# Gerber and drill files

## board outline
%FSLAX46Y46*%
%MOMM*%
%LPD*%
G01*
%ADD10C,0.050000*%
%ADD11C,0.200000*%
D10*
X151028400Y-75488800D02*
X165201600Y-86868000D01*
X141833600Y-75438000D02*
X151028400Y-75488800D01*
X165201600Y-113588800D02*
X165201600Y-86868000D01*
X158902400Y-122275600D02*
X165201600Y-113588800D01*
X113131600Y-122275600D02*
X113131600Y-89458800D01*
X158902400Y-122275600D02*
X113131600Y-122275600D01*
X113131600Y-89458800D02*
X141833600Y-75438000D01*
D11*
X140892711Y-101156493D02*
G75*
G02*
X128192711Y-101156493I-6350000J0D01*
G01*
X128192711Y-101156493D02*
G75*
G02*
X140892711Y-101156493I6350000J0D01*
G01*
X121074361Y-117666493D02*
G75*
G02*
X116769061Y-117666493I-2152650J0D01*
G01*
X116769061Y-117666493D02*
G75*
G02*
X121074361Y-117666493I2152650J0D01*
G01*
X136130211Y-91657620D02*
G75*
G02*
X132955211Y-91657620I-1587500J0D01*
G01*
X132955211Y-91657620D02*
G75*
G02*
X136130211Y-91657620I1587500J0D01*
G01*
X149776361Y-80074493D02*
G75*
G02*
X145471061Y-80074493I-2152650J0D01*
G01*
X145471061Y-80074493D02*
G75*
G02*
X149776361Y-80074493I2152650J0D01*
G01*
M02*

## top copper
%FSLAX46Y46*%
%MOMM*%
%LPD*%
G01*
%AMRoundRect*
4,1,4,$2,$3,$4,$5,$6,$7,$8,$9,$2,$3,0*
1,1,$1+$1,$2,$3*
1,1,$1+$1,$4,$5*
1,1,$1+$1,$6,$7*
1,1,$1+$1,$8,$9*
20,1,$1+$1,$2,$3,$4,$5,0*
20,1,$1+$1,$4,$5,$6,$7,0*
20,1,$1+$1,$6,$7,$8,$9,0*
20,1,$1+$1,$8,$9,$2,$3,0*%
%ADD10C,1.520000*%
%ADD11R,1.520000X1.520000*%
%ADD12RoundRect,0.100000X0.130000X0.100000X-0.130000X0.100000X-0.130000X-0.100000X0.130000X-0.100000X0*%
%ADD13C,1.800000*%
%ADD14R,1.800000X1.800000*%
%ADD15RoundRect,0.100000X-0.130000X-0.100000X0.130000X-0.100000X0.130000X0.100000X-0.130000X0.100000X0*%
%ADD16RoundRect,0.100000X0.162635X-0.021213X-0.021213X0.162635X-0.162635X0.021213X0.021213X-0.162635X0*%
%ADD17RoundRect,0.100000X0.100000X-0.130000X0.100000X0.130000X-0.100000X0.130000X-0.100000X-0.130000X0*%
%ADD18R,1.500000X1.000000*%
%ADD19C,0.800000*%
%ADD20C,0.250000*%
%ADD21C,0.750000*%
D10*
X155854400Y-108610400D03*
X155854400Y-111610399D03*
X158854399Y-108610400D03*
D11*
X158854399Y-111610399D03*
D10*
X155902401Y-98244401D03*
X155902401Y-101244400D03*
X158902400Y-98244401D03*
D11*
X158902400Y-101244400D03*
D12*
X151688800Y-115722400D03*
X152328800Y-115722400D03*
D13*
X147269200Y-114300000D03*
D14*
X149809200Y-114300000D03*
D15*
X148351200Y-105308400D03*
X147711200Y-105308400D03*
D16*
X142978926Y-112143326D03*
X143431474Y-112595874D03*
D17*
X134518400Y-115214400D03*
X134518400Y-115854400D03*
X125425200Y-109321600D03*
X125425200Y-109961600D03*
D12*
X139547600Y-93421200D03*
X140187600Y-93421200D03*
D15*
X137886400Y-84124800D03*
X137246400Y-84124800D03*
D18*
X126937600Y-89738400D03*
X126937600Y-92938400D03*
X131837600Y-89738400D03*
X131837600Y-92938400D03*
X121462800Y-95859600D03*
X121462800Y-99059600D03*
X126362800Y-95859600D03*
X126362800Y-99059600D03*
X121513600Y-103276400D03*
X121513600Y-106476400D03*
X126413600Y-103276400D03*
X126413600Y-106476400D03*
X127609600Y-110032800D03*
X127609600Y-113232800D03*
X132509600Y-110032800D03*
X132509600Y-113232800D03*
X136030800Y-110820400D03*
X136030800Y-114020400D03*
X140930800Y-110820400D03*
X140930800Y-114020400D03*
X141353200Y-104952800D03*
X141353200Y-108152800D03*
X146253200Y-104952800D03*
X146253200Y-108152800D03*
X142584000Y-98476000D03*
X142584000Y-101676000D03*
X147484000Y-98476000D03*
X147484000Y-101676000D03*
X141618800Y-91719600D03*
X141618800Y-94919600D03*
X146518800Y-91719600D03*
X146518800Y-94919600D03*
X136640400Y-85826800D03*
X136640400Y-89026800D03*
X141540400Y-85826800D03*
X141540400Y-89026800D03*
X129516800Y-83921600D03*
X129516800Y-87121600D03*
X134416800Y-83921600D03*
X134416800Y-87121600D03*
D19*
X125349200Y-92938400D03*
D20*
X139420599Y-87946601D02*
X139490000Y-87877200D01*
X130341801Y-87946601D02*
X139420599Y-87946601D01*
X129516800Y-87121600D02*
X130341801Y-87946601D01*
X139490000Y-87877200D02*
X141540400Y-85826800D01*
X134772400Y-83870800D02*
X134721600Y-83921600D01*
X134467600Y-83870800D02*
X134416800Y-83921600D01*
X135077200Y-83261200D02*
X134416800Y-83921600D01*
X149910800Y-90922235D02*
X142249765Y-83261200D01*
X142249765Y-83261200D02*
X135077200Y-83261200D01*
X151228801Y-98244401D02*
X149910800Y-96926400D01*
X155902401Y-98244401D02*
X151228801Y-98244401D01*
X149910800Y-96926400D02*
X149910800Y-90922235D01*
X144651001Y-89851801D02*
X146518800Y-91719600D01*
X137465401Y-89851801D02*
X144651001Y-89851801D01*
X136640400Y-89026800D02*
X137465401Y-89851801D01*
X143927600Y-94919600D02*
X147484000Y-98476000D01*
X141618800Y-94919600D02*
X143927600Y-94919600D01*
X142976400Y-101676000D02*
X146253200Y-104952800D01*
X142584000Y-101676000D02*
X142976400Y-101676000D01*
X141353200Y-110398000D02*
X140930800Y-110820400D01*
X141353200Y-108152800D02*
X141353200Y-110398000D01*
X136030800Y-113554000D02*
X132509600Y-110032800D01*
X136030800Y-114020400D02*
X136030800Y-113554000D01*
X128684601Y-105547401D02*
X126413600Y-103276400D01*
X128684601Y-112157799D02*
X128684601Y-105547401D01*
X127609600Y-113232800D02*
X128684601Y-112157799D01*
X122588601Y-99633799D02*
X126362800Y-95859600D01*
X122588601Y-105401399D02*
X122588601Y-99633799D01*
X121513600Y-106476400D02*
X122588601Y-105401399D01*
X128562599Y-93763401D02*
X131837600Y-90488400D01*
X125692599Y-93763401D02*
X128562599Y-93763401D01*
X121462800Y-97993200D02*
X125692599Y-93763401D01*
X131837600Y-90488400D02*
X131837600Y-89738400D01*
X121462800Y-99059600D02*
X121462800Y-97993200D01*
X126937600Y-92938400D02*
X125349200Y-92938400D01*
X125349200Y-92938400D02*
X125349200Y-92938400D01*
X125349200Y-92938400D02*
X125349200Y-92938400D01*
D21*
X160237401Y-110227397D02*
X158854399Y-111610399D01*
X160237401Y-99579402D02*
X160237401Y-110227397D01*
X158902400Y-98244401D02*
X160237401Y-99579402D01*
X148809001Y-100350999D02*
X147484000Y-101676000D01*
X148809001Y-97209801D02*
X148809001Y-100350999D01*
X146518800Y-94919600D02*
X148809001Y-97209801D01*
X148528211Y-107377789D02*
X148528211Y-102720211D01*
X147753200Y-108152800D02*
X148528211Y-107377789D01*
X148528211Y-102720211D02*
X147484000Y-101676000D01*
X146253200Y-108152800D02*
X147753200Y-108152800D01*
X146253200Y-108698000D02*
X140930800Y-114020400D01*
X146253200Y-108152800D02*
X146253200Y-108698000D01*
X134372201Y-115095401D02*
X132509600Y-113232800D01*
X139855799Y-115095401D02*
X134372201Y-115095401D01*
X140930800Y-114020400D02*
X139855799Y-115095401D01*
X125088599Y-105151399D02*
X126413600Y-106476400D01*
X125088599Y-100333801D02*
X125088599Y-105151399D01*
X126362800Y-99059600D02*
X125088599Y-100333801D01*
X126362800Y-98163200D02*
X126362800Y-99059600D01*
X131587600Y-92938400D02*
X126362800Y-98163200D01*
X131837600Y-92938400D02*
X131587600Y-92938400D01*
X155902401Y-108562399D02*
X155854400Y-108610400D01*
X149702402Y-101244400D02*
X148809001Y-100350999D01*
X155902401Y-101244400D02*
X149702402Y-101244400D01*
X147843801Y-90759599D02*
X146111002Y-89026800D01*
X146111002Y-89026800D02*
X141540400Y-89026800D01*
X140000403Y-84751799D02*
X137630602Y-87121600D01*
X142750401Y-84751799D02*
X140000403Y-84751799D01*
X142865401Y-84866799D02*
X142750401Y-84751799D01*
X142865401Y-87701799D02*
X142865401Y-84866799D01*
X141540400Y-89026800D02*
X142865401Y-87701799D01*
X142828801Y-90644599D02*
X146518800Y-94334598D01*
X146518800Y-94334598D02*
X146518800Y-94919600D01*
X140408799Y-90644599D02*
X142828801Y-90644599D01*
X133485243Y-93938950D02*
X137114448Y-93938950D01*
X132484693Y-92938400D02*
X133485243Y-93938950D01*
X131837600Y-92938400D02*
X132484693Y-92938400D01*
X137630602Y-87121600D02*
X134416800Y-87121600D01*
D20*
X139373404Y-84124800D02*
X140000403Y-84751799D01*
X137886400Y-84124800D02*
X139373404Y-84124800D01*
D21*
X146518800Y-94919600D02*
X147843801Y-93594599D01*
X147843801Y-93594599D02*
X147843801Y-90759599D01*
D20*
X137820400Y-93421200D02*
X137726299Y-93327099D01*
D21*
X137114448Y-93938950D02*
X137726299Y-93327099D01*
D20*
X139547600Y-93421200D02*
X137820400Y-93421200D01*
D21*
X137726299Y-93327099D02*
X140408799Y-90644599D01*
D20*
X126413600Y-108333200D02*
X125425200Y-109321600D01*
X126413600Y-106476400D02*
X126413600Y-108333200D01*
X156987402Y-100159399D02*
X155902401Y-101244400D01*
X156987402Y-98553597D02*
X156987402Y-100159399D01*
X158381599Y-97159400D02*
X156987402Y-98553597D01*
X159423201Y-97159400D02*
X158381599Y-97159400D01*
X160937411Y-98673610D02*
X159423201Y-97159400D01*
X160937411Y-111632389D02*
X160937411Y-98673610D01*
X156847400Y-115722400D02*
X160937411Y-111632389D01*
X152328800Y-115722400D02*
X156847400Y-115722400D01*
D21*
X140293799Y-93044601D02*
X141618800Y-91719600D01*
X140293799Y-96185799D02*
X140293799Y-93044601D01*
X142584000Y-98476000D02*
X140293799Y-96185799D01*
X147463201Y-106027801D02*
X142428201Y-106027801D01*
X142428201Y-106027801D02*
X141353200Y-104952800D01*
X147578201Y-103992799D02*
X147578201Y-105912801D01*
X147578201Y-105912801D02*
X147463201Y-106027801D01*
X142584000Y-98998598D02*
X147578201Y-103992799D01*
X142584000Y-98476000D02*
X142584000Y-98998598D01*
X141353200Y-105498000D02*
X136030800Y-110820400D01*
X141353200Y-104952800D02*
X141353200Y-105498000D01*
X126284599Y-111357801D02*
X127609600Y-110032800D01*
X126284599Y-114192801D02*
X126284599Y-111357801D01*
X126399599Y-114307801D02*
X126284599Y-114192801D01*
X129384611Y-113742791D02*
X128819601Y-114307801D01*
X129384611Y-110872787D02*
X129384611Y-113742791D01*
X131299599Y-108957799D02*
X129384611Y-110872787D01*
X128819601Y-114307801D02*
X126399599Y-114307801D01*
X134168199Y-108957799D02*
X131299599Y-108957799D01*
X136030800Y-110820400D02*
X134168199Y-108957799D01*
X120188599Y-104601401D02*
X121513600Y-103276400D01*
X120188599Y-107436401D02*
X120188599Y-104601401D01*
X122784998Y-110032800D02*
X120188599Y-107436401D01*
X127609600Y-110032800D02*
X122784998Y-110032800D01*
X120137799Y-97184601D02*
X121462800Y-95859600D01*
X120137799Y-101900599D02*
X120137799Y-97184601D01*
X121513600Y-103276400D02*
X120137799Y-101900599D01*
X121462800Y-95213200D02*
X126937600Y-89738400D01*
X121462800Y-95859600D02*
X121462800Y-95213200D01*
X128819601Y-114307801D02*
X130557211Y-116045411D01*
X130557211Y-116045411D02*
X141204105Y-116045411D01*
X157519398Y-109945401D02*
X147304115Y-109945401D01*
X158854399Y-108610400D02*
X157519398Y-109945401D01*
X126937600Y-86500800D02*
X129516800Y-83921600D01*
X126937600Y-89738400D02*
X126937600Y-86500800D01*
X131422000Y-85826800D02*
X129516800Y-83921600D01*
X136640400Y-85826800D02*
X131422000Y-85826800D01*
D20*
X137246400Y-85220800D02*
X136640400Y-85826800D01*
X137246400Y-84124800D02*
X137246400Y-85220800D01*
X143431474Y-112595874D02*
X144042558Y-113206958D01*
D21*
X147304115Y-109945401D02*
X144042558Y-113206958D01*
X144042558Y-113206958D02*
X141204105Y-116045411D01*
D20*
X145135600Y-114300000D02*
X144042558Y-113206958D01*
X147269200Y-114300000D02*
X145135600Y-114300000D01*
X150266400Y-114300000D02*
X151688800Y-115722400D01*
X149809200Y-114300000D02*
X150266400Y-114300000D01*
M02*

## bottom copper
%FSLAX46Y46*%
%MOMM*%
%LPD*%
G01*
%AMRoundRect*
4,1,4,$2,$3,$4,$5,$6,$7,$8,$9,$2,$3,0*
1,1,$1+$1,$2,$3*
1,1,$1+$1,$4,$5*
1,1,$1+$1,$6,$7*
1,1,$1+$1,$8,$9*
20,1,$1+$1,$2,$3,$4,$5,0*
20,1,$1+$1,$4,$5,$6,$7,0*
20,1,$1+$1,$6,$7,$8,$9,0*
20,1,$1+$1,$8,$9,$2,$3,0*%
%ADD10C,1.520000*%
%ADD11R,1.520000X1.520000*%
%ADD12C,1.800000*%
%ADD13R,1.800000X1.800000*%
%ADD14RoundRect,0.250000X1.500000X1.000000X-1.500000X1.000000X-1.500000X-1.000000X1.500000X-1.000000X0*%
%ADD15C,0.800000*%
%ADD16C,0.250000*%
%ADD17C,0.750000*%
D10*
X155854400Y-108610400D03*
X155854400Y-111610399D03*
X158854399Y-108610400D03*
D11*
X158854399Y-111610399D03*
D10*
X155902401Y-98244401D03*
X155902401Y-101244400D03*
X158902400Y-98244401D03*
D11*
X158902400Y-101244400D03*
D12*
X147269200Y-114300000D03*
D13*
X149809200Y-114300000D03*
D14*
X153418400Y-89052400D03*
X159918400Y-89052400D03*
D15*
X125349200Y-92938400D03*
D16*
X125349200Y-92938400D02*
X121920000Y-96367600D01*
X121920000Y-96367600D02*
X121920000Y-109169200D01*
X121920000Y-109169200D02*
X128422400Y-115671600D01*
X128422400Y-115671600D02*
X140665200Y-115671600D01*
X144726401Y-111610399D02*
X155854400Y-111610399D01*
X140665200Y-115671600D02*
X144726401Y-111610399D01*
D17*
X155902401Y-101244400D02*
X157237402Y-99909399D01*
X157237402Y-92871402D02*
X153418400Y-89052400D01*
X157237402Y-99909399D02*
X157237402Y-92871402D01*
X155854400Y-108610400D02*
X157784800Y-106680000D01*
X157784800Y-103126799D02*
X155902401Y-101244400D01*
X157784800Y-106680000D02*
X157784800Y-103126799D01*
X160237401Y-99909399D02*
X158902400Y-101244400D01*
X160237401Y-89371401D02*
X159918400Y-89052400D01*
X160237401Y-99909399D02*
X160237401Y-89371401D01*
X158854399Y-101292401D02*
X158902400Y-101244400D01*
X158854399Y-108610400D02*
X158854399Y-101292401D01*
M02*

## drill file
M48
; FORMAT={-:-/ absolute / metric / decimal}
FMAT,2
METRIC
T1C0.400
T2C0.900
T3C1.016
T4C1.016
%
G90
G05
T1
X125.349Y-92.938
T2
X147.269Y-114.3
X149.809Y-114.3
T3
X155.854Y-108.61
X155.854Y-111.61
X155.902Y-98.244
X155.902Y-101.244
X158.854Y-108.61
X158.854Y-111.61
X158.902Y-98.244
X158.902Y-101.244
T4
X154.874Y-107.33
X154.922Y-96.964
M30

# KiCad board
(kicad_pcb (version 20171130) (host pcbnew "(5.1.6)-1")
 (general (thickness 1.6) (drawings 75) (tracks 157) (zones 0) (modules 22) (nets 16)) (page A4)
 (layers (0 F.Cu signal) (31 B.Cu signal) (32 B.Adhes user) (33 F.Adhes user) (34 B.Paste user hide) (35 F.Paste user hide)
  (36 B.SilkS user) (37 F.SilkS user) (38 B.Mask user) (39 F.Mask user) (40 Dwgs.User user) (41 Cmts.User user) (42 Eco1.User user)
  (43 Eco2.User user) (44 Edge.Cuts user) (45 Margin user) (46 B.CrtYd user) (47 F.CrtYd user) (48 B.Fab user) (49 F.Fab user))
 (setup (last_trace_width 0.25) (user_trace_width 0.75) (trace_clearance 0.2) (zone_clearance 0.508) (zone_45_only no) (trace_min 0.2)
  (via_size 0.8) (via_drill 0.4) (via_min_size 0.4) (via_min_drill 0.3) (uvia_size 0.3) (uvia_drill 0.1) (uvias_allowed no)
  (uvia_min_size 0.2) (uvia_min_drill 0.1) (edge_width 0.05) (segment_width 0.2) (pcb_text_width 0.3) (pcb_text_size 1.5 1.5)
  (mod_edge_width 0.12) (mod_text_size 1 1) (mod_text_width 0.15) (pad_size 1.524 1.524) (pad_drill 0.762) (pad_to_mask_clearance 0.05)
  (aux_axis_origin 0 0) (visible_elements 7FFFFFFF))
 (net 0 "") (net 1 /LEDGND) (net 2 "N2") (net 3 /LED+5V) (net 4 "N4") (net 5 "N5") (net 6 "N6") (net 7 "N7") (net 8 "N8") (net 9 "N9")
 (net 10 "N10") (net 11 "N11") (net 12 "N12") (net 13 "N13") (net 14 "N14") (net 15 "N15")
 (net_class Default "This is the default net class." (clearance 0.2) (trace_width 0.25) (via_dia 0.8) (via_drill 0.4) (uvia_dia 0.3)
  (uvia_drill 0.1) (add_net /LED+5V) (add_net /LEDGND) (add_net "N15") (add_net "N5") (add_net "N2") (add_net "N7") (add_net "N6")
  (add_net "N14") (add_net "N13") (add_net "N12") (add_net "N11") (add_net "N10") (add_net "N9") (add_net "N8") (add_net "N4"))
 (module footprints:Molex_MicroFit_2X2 (layer B.Cu) (at 158.854399 111.610399 270)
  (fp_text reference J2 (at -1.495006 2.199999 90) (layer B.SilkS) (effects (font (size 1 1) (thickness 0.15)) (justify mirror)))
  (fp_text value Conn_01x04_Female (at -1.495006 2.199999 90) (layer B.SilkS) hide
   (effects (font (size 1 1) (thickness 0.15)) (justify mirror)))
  (pad 5 np_thru_hole circle (at -4.279999 3.98 270) (size 1.02 1.02) (drill 1.016) (layers))
  (pad 4 thru_hole circle (at -2.999999 2.999999 270) (size 1.52 1.52) (drill 1.016) (layers *.Cu *.Mask) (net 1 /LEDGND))
  (pad 3 thru_hole circle (at 0 2.999999 180) (size 1.52 1.52) (drill 1.016) (layers *.Cu *.Mask) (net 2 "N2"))
  (pad 2 thru_hole circle (at -2.999999 0 270) (size 1.52 1.52) (drill 1.016) (layers *.Cu *.Mask) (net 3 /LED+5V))
  (pad 1 thru_hole rect (at 0 0 180) (size 1.52 1.52) (drill 1.016) (layers *.Cu *.Mask) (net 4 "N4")))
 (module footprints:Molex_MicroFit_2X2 (layer B.Cu) (at 158.9024 101.2444 270)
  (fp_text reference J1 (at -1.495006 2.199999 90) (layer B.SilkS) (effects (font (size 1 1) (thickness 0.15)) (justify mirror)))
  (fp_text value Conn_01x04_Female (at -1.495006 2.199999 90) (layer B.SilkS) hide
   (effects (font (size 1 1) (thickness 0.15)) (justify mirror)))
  (pad 5 np_thru_hole circle (at -4.279999 3.98 270) (size 1.02 1.02) (drill 1.016) (layers))
  (pad 4 thru_hole circle (at -2.999999 2.999999 270) (size 1.52 1.52) (drill 1.016) (layers *.Cu *.Mask) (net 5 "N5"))
  (pad 3 thru_hole circle (at 0 2.999999 180) (size 1.52 1.52) (drill 1.016) (layers *.Cu *.Mask) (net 1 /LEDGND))
  (pad 2 thru_hole circle (at -2.999999 0 270) (size 1.52 1.52) (drill 1.016) (layers *.Cu *.Mask) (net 4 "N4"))
  (pad 1 thru_hole rect (at 0 0 180) (size 1.52 1.52) (drill 1.016) (layers *.Cu *.Mask) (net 3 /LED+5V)))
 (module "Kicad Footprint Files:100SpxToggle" (layer F.Cu) (at 145.4912 101.092)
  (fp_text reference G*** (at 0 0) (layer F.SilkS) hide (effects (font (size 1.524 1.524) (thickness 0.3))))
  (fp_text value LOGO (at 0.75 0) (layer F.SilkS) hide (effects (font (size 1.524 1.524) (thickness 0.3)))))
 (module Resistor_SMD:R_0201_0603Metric (layer F.Cu) (at 152.0088 115.7224 180)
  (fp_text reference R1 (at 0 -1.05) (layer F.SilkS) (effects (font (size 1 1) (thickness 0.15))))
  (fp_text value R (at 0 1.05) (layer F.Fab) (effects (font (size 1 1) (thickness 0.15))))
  (pad 2 smd roundrect (at 0.32 0 180) (size 0.46 0.4) (layers F.Cu F.Mask) (roundrect_rratio 0.25) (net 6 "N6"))
  (pad 1 smd roundrect (at -0.32 0 180) (size 0.46 0.4) (layers F.Cu F.Mask) (roundrect_rratio 0.25) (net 1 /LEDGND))
  (pad "" smd roundrect (at 0.345 0 180) (size 0.318 0.36) (layers F.Paste) (roundrect_rratio 0.25))
  (pad "" smd roundrect (at -0.345 0 180) (size 0.318 0.36) (layers F.Paste) (roundrect_rratio 0.25)))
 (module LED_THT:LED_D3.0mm (layer B.Cu) (at 149.8092 114.3 180)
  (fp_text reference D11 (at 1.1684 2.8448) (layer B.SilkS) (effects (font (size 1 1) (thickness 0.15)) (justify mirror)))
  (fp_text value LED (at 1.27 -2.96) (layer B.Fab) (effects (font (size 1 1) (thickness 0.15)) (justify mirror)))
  (pad 2 thru_hole circle (at 2.54 0 180) (size 1.8 1.8) (drill 0.9) (layers *.Cu *.Mask) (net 3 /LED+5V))
  (pad 1 thru_hole rect (at 0 0 180) (size 1.8 1.8) (drill 0.9) (layers *.Cu *.Mask) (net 6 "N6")))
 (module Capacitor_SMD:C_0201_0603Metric (layer F.Cu) (at 148.0312 105.3084)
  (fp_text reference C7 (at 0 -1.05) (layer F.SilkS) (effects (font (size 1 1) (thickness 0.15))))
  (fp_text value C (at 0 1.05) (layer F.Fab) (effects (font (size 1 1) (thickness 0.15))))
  (pad 2 smd roundrect (at 0.32 0) (size 0.46 0.4) (layers F.Cu F.Mask) (roundrect_rratio 0.25) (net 1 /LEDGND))
  (pad 1 smd roundrect (at -0.32 0) (size 0.46 0.4) (layers F.Cu F.Mask) (roundrect_rratio 0.25) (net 3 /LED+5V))
  (pad "" smd roundrect (at 0.345 0) (size 0.318 0.36) (layers F.Paste) (roundrect_rratio 0.25))
  (pad "" smd roundrect (at -0.345 0) (size 0.318 0.36) (layers F.Paste) (roundrect_rratio 0.25)))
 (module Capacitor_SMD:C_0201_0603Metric (layer F.Cu) (at 143.2052 112.3696 135)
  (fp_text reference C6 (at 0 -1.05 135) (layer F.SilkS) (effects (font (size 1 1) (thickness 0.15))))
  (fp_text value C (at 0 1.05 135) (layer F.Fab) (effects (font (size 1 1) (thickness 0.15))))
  (pad 2 smd roundrect (at 0.32 0 135) (size 0.46 0.4) (layers F.Cu F.Mask) (roundrect_rratio 0.25) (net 1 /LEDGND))
  (pad 1 smd roundrect (at -0.32 0 135) (size 0.46 0.4) (layers F.Cu F.Mask) (roundrect_rratio 0.25) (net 3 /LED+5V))
  (pad "" smd roundrect (at 0.345 0 135) (size 0.318 0.36) (layers F.Paste) (roundrect_rratio 0.25))
  (pad "" smd roundrect (at -0.345 0 135) (size 0.318 0.36) (layers F.Paste) (roundrect_rratio 0.25)))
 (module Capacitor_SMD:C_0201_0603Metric (layer F.Cu) (at 134.5184 115.5344 90)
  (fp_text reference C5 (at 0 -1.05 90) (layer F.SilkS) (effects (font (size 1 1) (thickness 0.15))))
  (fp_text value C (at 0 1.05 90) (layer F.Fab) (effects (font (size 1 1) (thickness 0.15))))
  (pad 2 smd roundrect (at 0.32 0 90) (size 0.46 0.4) (layers F.Cu F.Mask) (roundrect_rratio 0.25) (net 1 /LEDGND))
  (pad 1 smd roundrect (at -0.32 0 90) (size 0.46 0.4) (layers F.Cu F.Mask) (roundrect_rratio 0.25) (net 3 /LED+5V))
  (pad "" smd roundrect (at 0.345 0 90) (size 0.318 0.36) (layers F.Paste) (roundrect_rratio 0.25))
  (pad "" smd roundrect (at -0.345 0 90) (size 0.318 0.36) (layers F.Paste) (roundrect_rratio 0.25)))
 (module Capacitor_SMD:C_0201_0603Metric (layer F.Cu) (at 125.4252 109.6416 90)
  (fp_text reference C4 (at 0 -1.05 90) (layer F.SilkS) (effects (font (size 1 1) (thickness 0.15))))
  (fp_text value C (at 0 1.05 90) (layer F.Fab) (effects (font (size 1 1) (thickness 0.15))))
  (pad 2 smd roundrect (at 0.32 0 90) (size 0.46 0.4) (layers F.Cu F.Mask) (roundrect_rratio 0.25) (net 1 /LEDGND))
  (pad 1 smd roundrect (at -0.32 0 90) (size 0.46 0.4) (layers F.Cu F.Mask) (roundrect_rratio 0.25) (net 3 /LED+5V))
  (pad "" smd roundrect (at 0.345 0 90) (size 0.318 0.36) (layers F.Paste) (roundrect_rratio 0.25))
  (pad "" smd roundrect (at -0.345 0 90) (size 0.318 0.36) (layers F.Paste) (roundrect_rratio 0.25)))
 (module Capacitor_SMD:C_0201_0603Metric (layer F.Cu) (at 139.8676 93.4212 180)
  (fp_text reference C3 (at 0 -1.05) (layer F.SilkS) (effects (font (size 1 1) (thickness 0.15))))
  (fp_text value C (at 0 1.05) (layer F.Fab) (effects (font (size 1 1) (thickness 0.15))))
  (pad 2 smd roundrect (at 0.32 0 180) (size 0.46 0.4) (layers F.Cu F.Mask) (roundrect_rratio 0.25) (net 1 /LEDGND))
  (pad 1 smd roundrect (at -0.32 0 180) (size 0.46 0.4) (layers F.Cu F.Mask) (roundrect_rratio 0.25) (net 3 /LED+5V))
  (pad "" smd roundrect (at 0.345 0 180) (size 0.318 0.36) (layers F.Paste) (roundrect_rratio 0.25))
  (pad "" smd roundrect (at -0.345 0 180) (size 0.318 0.36) (layers F.Paste) (roundrect_rratio 0.25)))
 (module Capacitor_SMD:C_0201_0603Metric (layer F.Cu) (at 137.5664 84.1248)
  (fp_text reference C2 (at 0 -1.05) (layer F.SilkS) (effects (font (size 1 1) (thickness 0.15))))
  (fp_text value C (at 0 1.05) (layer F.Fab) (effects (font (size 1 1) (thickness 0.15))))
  (pad 2 smd roundrect (at 0.32 0) (size 0.46 0.4) (layers F.Cu F.Mask) (roundrect_rratio 0.25) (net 1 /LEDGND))
  (pad 1 smd roundrect (at -0.32 0) (size 0.46 0.4) (layers F.Cu F.Mask) (roundrect_rratio 0.25) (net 3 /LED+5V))
  (pad "" smd roundrect (at 0.345 0) (size 0.318 0.36) (layers F.Paste) (roundrect_rratio 0.25))
  (pad "" smd roundrect (at -0.345 0) (size 0.318 0.36) (layers F.Paste) (roundrect_rratio 0.25)))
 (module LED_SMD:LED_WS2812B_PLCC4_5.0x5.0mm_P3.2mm (layer F.Cu) (at 129.3876 91.3384)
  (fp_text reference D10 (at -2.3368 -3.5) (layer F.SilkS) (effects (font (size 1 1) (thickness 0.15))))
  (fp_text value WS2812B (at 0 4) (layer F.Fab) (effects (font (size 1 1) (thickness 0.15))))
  (pad 1 smd rect (at -2.45 -1.6) (size 1.5 1) (layers F.Cu F.Paste F.Mask) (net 3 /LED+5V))
  (pad 2 smd rect (at -2.45 1.6) (size 1.5 1) (layers F.Cu F.Paste F.Mask) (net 2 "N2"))
  (pad 4 smd rect (at 2.45 -1.6) (size 1.5 1) (layers F.Cu F.Paste F.Mask) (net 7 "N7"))
  (pad 3 smd rect (at 2.45 1.6) (size 1.5 1) (layers F.Cu F.Paste F.Mask) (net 1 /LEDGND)))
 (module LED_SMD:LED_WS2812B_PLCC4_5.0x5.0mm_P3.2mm (layer F.Cu) (at 123.9128 97.4596)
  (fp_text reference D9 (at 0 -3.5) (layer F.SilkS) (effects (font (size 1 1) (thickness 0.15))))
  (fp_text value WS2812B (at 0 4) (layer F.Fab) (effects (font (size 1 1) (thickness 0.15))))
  (pad 1 smd rect (at -2.45 -1.6) (size 1.5 1) (layers F.Cu F.Paste F.Mask) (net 3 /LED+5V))
  (pad 2 smd rect (at -2.45 1.6) (size 1.5 1) (layers F.Cu F.Paste F.Mask) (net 7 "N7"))
  (pad 4 smd rect (at 2.45 -1.6) (size 1.5 1) (layers F.Cu F.Paste F.Mask) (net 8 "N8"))
  (pad 3 smd rect (at 2.45 1.6) (size 1.5 1) (layers F.Cu F.Paste F.Mask) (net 1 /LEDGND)))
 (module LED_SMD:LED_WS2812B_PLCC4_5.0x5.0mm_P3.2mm (layer F.Cu) (at 123.9636 104.8764)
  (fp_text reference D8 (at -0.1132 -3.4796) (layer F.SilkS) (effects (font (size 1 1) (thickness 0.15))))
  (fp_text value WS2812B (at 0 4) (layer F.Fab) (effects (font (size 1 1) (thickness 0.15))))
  (pad 1 smd rect (at -2.45 -1.6) (size 1.5 1) (layers F.Cu F.Paste F.Mask) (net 3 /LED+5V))
  (pad 2 smd rect (at -2.45 1.6) (size 1.5 1) (layers F.Cu F.Paste F.Mask) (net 8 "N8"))
  (pad 4 smd rect (at 2.45 -1.6) (size 1.5 1) (layers F.Cu F.Paste F.Mask) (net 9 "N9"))
  (pad 3 smd rect (at 2.45 1.6) (size 1.5 1) (layers F.Cu F.Paste F.Mask) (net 1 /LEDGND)))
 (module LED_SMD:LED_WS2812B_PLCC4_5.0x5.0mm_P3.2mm (layer F.Cu) (at 130.0596 111.6328)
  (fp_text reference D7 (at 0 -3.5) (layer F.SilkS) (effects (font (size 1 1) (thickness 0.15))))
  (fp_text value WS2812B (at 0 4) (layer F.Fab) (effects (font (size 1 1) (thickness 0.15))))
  (pad 1 smd rect (at -2.45 -1.6) (size 1.5 1) (layers F.Cu F.Paste F.Mask) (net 3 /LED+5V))
  (pad 2 smd rect (at -2.45 1.6) (size 1.5 1) (layers F.Cu F.Paste F.Mask) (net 9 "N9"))
  (pad 4 smd rect (at 2.45 -1.6) (size 1.5 1) (layers F.Cu F.Paste F.Mask) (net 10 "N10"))
  (pad 3 smd rect (at 2.45 1.6) (size 1.5 1) (layers F.Cu F.Paste F.Mask) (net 1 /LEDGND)))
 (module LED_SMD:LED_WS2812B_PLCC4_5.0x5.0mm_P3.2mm (layer F.Cu) (at 138.4808 112.4204)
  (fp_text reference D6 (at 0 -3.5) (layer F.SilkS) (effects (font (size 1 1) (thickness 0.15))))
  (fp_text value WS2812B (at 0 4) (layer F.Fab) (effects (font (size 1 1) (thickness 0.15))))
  (pad 1 smd rect (at -2.45 -1.6) (size 1.5 1) (layers F.Cu F.Paste F.Mask) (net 3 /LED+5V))
  (pad 2 smd rect (at -2.45 1.6) (size 1.5 1) (layers F.Cu F.Paste F.Mask) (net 10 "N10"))
  (pad 4 smd rect (at 2.45 -1.6) (size 1.5 1) (layers F.Cu F.Paste F.Mask) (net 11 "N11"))
  (pad 3 smd rect (at 2.45 1.6) (size 1.5 1) (layers F.Cu F.Paste F.Mask) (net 1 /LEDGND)))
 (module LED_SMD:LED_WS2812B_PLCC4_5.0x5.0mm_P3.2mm (layer F.Cu) (at 143.8032 106.5528)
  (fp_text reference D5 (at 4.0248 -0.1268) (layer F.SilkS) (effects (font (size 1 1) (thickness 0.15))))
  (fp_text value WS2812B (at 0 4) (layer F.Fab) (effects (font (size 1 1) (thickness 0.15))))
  (pad 1 smd rect (at -2.45 -1.6) (size 1.5 1) (layers F.Cu F.Paste F.Mask) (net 3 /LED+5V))
  (pad 2 smd rect (at -2.45 1.6) (size 1.5 1) (layers F.Cu F.Paste F.Mask) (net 11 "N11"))
  (pad 4 smd rect (at 2.45 -1.6) (size 1.5 1) (layers F.Cu F.Paste F.Mask) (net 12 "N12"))
  (pad 3 smd rect (at 2.45 1.6) (size 1.5 1) (layers F.Cu F.Paste F.Mask) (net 1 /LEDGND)))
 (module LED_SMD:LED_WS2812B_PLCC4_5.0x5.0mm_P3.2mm (layer F.Cu) (at 145.034 100.076)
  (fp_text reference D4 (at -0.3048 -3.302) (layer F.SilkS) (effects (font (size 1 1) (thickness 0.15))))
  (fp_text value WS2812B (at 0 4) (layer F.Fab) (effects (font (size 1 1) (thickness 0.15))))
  (pad 1 smd rect (at -2.45 -1.6) (size 1.5 1) (layers F.Cu F.Paste F.Mask) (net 3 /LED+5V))
  (pad 2 smd rect (at -2.45 1.6) (size 1.5 1) (layers F.Cu F.Paste F.Mask) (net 12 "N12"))
  (pad 4 smd rect (at 2.45 -1.6) (size 1.5 1) (layers F.Cu F.Paste F.Mask) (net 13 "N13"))
  (pad 3 smd rect (at 2.45 1.6) (size 1.5 1) (layers F.Cu F.Paste F.Mask) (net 1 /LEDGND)))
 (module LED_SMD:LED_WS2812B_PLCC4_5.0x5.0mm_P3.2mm (layer F.Cu) (at 144.0688 93.3196)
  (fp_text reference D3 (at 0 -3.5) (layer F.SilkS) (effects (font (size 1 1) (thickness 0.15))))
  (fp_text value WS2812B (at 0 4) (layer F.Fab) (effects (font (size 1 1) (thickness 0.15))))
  (pad 1 smd rect (at -2.45 -1.6) (size 1.5 1) (layers F.Cu F.Paste F.Mask) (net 3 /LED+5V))
  (pad 2 smd rect (at -2.45 1.6) (size 1.5 1) (layers F.Cu F.Paste F.Mask) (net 13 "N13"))
  (pad 4 smd rect (at 2.45 -1.6) (size 1.5 1) (layers F.Cu F.Paste F.Mask) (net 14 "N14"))
  (pad 3 smd rect (at 2.45 1.6) (size 1.5 1) (layers F.Cu F.Paste F.Mask) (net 1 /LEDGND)))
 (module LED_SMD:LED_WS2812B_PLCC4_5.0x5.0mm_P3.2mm (layer F.Cu) (at 139.0904 87.4268)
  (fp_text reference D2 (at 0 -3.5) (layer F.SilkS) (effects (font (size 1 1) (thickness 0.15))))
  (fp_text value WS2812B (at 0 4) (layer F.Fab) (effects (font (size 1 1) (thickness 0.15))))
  (pad 1 smd rect (at -2.45 -1.6) (size 1.5 1) (layers F.Cu F.Paste F.Mask) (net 3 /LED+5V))
  (pad 2 smd rect (at -2.45 1.6) (size 1.5 1) (layers F.Cu F.Paste F.Mask) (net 14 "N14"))
  (pad 4 smd rect (at 2.45 -1.6) (size 1.5 1) (layers F.Cu F.Paste F.Mask) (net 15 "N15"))
  (pad 3 smd rect (at 2.45 1.6) (size 1.5 1) (layers F.Cu F.Paste F.Mask) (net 1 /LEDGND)))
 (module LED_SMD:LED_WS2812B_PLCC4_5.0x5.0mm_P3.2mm (layer F.Cu) (at 131.9668 85.5216)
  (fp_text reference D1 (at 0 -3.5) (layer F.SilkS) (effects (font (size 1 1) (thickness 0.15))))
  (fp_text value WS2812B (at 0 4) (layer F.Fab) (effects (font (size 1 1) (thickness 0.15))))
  (pad 1 smd rect (at -2.45 -1.6) (size 1.5 1) (layers F.Cu F.Paste F.Mask) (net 3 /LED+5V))
  (pad 2 smd rect (at -2.45 1.6) (size 1.5 1) (layers F.Cu F.Paste F.Mask) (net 15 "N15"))
  (pad 4 smd rect (at 2.45 -1.6) (size 1.5 1) (layers F.Cu F.Paste F.Mask) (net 5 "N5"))
  (pad 3 smd rect (at 2.45 1.6) (size 1.5 1) (layers F.Cu F.Paste F.Mask) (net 1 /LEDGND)))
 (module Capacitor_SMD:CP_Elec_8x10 (layer B.Cu) (at 156.6684 89.0524 180)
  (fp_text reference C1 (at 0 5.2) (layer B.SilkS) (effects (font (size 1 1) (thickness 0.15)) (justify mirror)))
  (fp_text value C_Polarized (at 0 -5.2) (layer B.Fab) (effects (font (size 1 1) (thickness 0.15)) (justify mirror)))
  (pad 2 smd roundrect (at 3.25 0 180) (size 3.5 2.5) (layers B.Cu B.Paste B.Mask) (roundrect_rratio 0.1) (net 1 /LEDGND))
  (pad 1 smd roundrect (at -3.25 0 180) (size 3.5 2.5) (layers B.Cu B.Paste B.Mask) (roundrect_rratio 0.1) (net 3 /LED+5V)))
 (gr_line (start 151.0284 75.4888) (end 165.2016 86.868) (layer Edge.Cuts) (width 0.05))
 (gr_line (start 141.8336 75.438) (end 151.0284 75.4888) (layer Edge.Cuts) (width 0.05))
 (gr_line (start 165.2016 113.5888) (end 165.2016 86.868) (layer Edge.Cuts) (width 0.05))
 (gr_line (start 158.9024 122.2756) (end 165.2016 113.5888) (layer Edge.Cuts) (width 0.05))
 (gr_line (start 113.1316 122.2756) (end 113.1316 89.4588) (layer Edge.Cuts) (width 0.05))
 (gr_line (start 158.9024 122.2756) (end 113.1316 122.2756) (layer Edge.Cuts) (width 0.05))
 (gr_line (start 113.1316 89.4588) (end 141.8336 75.438) (layer Edge.Cuts) (width 0.05))
 (gr_circle (center 134.542711 101.156493) (end 140.892711 101.156493) (layer Edge.Cuts) (width 0.2))
 (gr_circle (center 118.921711 117.666493) (end 121.074361 117.666493) (layer Edge.Cuts) (width 0.2))
 (gr_circle (center 134.542711 91.65762) (end 136.130211 91.65762) (layer Edge.Cuts) (width 0.2))
 (gr_circle (center 147.623711 80.074493) (end 149.776361 80.074493) (layer Edge.Cuts) (width 0.2))
 (segment (start 139.420599 87.946601) (end 139.49 87.8772) (width 0.25) (layer F.Cu) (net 15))
 (segment (start 130.341801 87.946601) (end 139.420599 87.946601) (width 0.25) (layer F.Cu) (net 15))
 (segment (start 129.5168 87.1216) (end 130.341801 87.946601) (width 0.25) (layer F.Cu) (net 15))
 (segment (start 139.49 87.8772) (end 141.5404 85.8268) (width 0.25) (layer F.Cu) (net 15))
 (segment (start 134.7724 83.8708) (end 134.7216 83.9216) (width 0.25) (layer F.Cu) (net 5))
 (segment (start 134.4676 83.8708) (end 134.4168 83.9216) (width 0.25) (layer F.Cu) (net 5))
 (segment (start 135.0772 83.2612) (end 134.4168 83.9216) (width 0.25) (layer F.Cu) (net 5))
 (segment (start 149.9108 90.922235) (end 142.249765 83.2612) (width 0.25) (layer F.Cu) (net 5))
 (segment (start 142.249765 83.2612) (end 135.0772 83.2612) (width 0.25) (layer F.Cu) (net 5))
 (segment (start 151.228801 98.244401) (end 149.9108 96.9264) (width 0.25) (layer F.Cu) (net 5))
 (segment (start 155.902401 98.244401) (end 151.228801 98.244401) (width 0.25) (layer F.Cu) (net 5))
 (segment (start 149.9108 96.9264) (end 149.9108 90.922235) (width 0.25) (layer F.Cu) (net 5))
 (segment (start 144.651001 89.851801) (end 146.5188 91.7196) (width 0.25) (layer F.Cu) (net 14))
 (segment (start 137.465401 89.851801) (end 144.651001 89.851801) (width 0.25) (layer F.Cu) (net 14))
 (segment (start 136.6404 89.0268) (end 137.465401 89.851801) (width 0.25) (layer F.Cu) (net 14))
 (segment (start 143.9276 94.9196) (end 147.484 98.476) (width 0.25) (layer F.Cu) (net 13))
 (segment (start 141.6188 94.9196) (end 143.9276 94.9196) (width 0.25) (layer F.Cu) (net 13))
 (segment (start 142.9764 101.676) (end 146.2532 104.9528) (width 0.25) (layer F.Cu) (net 12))
 (segment (start 142.584 101.676) (end 142.9764 101.676) (width 0.25) (layer F.Cu) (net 12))
 (segment (start 141.3532 110.398) (end 140.9308 110.8204) (width 0.25) (layer F.Cu) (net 11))
 (segment (start 141.3532 108.1528) (end 141.3532 110.398) (width 0.25) (layer F.Cu) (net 11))
 (segment (start 136.0308 113.554) (end 132.5096 110.0328) (width 0.25) (layer F.Cu) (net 10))
 (segment (start 136.0308 114.0204) (end 136.0308 113.554) (width 0.25) (layer F.Cu) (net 10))
 (segment (start 128.684601 105.547401) (end 126.4136 103.2764) (width 0.25) (layer F.Cu) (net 9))
 (segment (start 128.684601 112.157799) (end 128.684601 105.547401) (width 0.25) (layer F.Cu) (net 9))
 (segment (start 127.6096 113.2328) (end 128.684601 112.157799) (width 0.25) (layer F.Cu) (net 9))
 (segment (start 122.588601 99.633799) (end 126.3628 95.8596) (width 0.25) (layer F.Cu) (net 8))
 (segment (start 122.588601 105.401399) (end 122.588601 99.633799) (width 0.25) (layer F.Cu) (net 8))
 (segment (start 121.5136 106.4764) (end 122.588601 105.401399) (width 0.25) (layer F.Cu) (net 8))
 (segment (start 128.562599 93.763401) (end 131.8376 90.4884) (width 0.25) (layer F.Cu) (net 7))
 (segment (start 125.692599 93.763401) (end 128.562599 93.763401) (width 0.25) (layer F.Cu) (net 7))
 (segment (start 121.4628 97.9932) (end 125.692599 93.763401) (width 0.25) (layer F.Cu) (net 7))
 (segment (start 131.8376 90.4884) (end 131.8376 89.7384) (width 0.25) (layer F.Cu) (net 7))
 (segment (start 121.4628 99.0596) (end 121.4628 97.9932) (width 0.25) (layer F.Cu) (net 7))
 (segment (start 126.9376 92.9384) (end 125.3492 92.9384) (width 0.25) (layer F.Cu) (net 2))
 (segment (start 125.3492 92.9384) (end 125.3492 92.9384) (width 0.25) (layer F.Cu) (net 2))
 (segment (start 125.3492 92.9384) (end 125.3492 92.9384) (width 0.25) (layer F.Cu) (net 2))
 (via (at 125.3492 92.9384) (size 0.8) (drill 0.4) (layers F.Cu B.Cu) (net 2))
 (segment (start 125.3492 92.9384) (end 121.92 96.3676) (width 0.25) (layer B.Cu) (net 2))
 (segment (start 121.92 96.3676) (end 121.92 109.1692) (width 0.25) (layer B.Cu) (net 2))
 (segment (start 121.92 109.1692) (end 128.4224 115.6716) (width 0.25) (layer B.Cu) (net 2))
 (segment (start 128.4224 115.6716) (end 140.6652 115.6716) (width 0.25) (layer B.Cu) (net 2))
 (segment (start 144.726401 111.610399) (end 155.8544 111.610399) (width 0.25) (layer B.Cu) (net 2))
 (segment (start 140.6652 115.6716) (end 144.726401 111.610399) (width 0.25) (layer B.Cu) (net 2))
 (segment (start 160.237401 110.227397) (end 158.854399 111.610399) (width 0.75) (layer F.Cu) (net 4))
 (segment (start 160.237401 99.579402) (end 160.237401 110.227397) (width 0.75) (layer F.Cu) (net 4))
 (segment (start 158.9024 98.244401) (end 160.237401 99.579402) (width 0.75) (layer F.Cu) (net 4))
 (segment (start 148.809001 100.350999) (end 147.484 101.676) (width 0.75) (layer F.Cu) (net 1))
 (segment (start 148.809001 97.209801) (end 148.809001 100.350999) (width 0.75) (layer F.Cu) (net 1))
 (segment (start 146.5188 94.9196) (end 148.809001 97.209801) (width 0.75) (layer F.Cu) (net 1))
 (segment (start 148.528211 107.377789) (end 148.528211 102.720211) (width 0.75) (layer F.Cu) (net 1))
 (segment (start 147.7532 108.1528) (end 148.528211 107.377789) (width 0.75) (layer F.Cu) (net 1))
 (segment (start 148.528211 102.720211) (end 147.484 101.676) (width 0.75) (layer F.Cu) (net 1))
 (segment (start 146.2532 108.1528) (end 147.7532 108.1528) (width 0.75) (layer F.Cu) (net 1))
 (segment (start 146.2532 108.698) (end 140.9308 114.0204) (width 0.75) (layer F.Cu) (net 1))
 (segment (start 146.2532 108.1528) (end 146.2532 108.698) (width 0.75) (layer F.Cu) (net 1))
 (segment (start 134.372201 115.095401) (end 132.5096 113.2328) (width 0.75) (layer F.Cu) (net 1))
 (segment (start 139.855799 115.095401) (end 134.372201 115.095401) (width 0.75) (layer F.Cu) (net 1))
 (segment (start 140.9308 114.0204) (end 139.855799 115.095401) (width 0.75) (layer F.Cu) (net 1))
 (segment (start 125.088599 105.151399) (end 126.4136 106.4764) (width 0.75) (layer F.Cu) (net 1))
 (segment (start 125.088599 100.333801) (end 125.088599 105.151399) (width 0.75) (layer F.Cu) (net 1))
 (segment (start 126.3628 99.0596) (end 125.088599 100.333801) (width 0.75) (layer F.Cu) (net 1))
 (segment (start 126.3628 98.1632) (end 126.3628 99.0596) (width 0.75) (layer F.Cu) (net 1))
 (segment (start 131.5876 92.9384) (end 126.3628 98.1632) (width 0.75) (layer F.Cu) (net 1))
 (segment (start 131.8376 92.9384) (end 131.5876 92.9384) (width 0.75) (layer F.Cu) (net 1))
 (segment (start 155.902401 108.562399) (end 155.8544 108.6104) (width 0.75) (layer F.Cu) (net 1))
 (segment (start 155.902401 101.2444) (end 157.237402 99.909399) (width 0.75) (layer B.Cu) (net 1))
 (segment (start 149.702402 101.2444) (end 148.809001 100.350999) (width 0.75) (layer F.Cu) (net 1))
 (segment (start 155.902401 101.2444) (end 149.702402 101.2444) (width 0.75) (layer F.Cu) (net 1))
 (segment (start 147.843801 90.759599) (end 146.111002 89.0268) (width 0.75) (layer F.Cu) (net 1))
 (segment (start 146.111002 89.0268) (end 141.5404 89.0268) (width 0.75) (layer F.Cu) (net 1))
 (segment (start 140.000403 84.751799) (end 137.630602 87.1216) (width 0.75) (layer F.Cu) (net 1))
 (segment (start 142.750401 84.751799) (end 140.000403 84.751799) (width 0.75) (layer F.Cu) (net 1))
 (segment (start 142.865401 84.866799) (end 142.750401 84.751799) (width 0.75) (layer F.Cu) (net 1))
 (segment (start 142.865401 87.701799) (end 142.865401 84.866799) (width 0.75) (layer F.Cu) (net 1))
 (segment (start 141.5404 89.0268) (end 142.865401 87.701799) (width 0.75) (layer F.Cu) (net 1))
 (segment (start 142.828801 90.644599) (end 146.5188 94.334598) (width 0.75) (layer F.Cu) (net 1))
 (segment (start 146.5188 94.334598) (end 146.5188 94.9196) (width 0.75) (layer F.Cu) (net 1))
 (segment (start 140.408799 90.644599) (end 142.828801 90.644599) (width 0.75) (layer F.Cu) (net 1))
 (segment (start 133.485243 93.93895) (end 137.114448 93.93895) (width 0.75) (layer F.Cu) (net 1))
 (segment (start 132.484693 92.9384) (end 133.485243 93.93895) (width 0.75) (layer F.Cu) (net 1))
 (segment (start 131.8376 92.9384) (end 132.484693 92.9384) (width 0.75) (layer F.Cu) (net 1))
 (segment (start 137.630602 87.1216) (end 134.4168 87.1216) (width 0.75) (layer F.Cu) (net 1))
 (segment (start 157.237402 92.871402) (end 153.4184 89.0524) (width 0.75) (layer B.Cu) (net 1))
 (segment (start 157.237402 99.909399) (end 157.237402 92.871402) (width 0.75) (layer B.Cu) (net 1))
 (segment (start 155.8544 108.6104) (end 157.7848 106.68) (width 0.75) (layer B.Cu) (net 1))
 (segment (start 157.7848 103.126799) (end 155.902401 101.2444) (width 0.75) (layer B.Cu) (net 1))
 (segment (start 157.7848 106.68) (end 157.7848 103.126799) (width 0.75) (layer B.Cu) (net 1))
 (segment (start 139.373404 84.1248) (end 140.000403 84.751799) (width 0.25) (layer F.Cu) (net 1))
 (segment (start 137.8864 84.1248) (end 139.373404 84.1248) (width 0.25) (layer F.Cu) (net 1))
 (segment (start 146.5188 94.9196) (end 147.843801 93.594599) (width 0.75) (layer F.Cu) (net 1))
 (segment (start 147.843801 93.594599) (end 147.843801 90.759599) (width 0.75) (layer F.Cu) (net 1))
 (segment (start 137.8204 93.4212) (end 137.726299 93.327099) (width 0.25) (layer F.Cu) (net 1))
 (segment (start 137.114448 93.93895) (end 137.726299 93.327099) (width 0.75) (layer F.Cu) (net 1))
 (segment (start 139.5476 93.4212) (end 137.8204 93.4212) (width 0.25) (layer F.Cu) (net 1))
 (segment (start 137.726299 93.327099) (end 140.408799 90.644599) (width 0.75) (layer F.Cu) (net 1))
 (segment (start 126.4136 108.3332) (end 125.4252 109.3216) (width 0.25) (layer F.Cu) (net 1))
 (segment (start 126.4136 106.4764) (end 126.4136 108.3332) (width 0.25) (layer F.Cu) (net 1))
 (segment (start 156.987402 100.159399) (end 155.902401 101.2444) (width 0.25) (layer F.Cu) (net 1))
 (segment (start 156.987402 98.553597) (end 156.987402 100.159399) (width 0.25) (layer F.Cu) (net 1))
 (segment (start 158.381599 97.1594) (end 156.987402 98.553597) (width 0.25) (layer F.Cu) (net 1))
 (segment (start 159.423201 97.1594) (end 158.381599 97.1594) (width 0.25) (layer F.Cu) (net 1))
 (segment (start 160.937411 98.67361) (end 159.423201 97.1594) (width 0.25) (layer F.Cu) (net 1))
 (segment (start 160.937411 111.632389) (end 160.937411 98.67361) (width 0.25) (layer F.Cu) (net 1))
 (segment (start 156.8474 115.7224) (end 160.937411 111.632389) (width 0.25) (layer F.Cu) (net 1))
 (segment (start 152.3288 115.7224) (end 156.8474 115.7224) (width 0.25) (layer F.Cu) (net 1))
 (segment (start 140.293799 93.044601) (end 141.6188 91.7196) (width 0.75) (layer F.Cu) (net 3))
 (segment (start 140.293799 96.185799) (end 140.293799 93.044601) (width 0.75) (layer F.Cu) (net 3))
 (segment (start 142.584 98.476) (end 140.293799 96.185799) (width 0.75) (layer F.Cu) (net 3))
 (segment (start 147.463201 106.027801) (end 142.428201 106.027801) (width 0.75) (layer F.Cu) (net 3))
 (segment (start 142.428201 106.027801) (end 141.3532 104.9528) (width 0.75) (layer F.Cu) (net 3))
 (segment (start 147.578201 103.992799) (end 147.578201 105.912801) (width 0.75) (layer F.Cu) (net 3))
 (segment (start 147.578201 105.912801) (end 147.463201 106.027801) (width 0.75) (layer F.Cu) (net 3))
 (segment (start 142.584 98.998598) (end 147.578201 103.992799) (width 0.75) (layer F.Cu) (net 3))
 (segment (start 142.584 98.476) (end 142.584 98.998598) (width 0.75) (layer F.Cu) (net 3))
 (segment (start 141.3532 105.498) (end 136.0308 110.8204) (width 0.75) (layer F.Cu) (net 3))
 (segment (start 141.3532 104.9528) (end 141.3532 105.498) (width 0.75) (layer F.Cu) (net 3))
 (segment (start 126.284599 111.357801) (end 127.6096 110.0328) (width 0.75) (layer F.Cu) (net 3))
 (segment (start 126.284599 114.192801) (end 126.284599 111.357801) (width 0.75) (layer F.Cu) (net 3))
 (segment (start 126.399599 114.307801) (end 126.284599 114.192801) (width 0.75) (layer F.Cu) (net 3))
 (segment (start 129.384611 113.742791) (end 128.819601 114.307801) (width 0.75) (layer F.Cu) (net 3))
 (segment (start 129.384611 110.872787) (end 129.384611 113.742791) (width 0.75) (layer F.Cu) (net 3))
 (segment (start 131.299599 108.957799) (end 129.384611 110.872787) (width 0.75) (layer F.Cu) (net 3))
 (segment (start 128.819601 114.307801) (end 126.399599 114.307801) (width 0.75) (layer F.Cu) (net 3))
 (segment (start 134.168199 108.957799) (end 131.299599 108.957799) (width 0.75) (layer F.Cu) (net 3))
 (segment (start 136.0308 110.8204) (end 134.168199 108.957799) (width 0.75) (layer F.Cu) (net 3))
 (segment (start 120.188599 104.601401) (end 121.5136 103.2764) (width 0.75) (layer F.Cu) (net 3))
 (segment (start 120.188599 107.436401) (end 120.188599 104.601401) (width 0.75) (layer F.Cu) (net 3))
 (segment (start 122.784998 110.0328) (end 120.188599 107.436401) (width 0.75) (layer F.Cu) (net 3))
 (segment (start 127.6096 110.0328) (end 122.784998 110.0328) (width 0.75) (layer F.Cu) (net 3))
 (segment (start 120.137799 97.184601) (end 121.4628 95.8596) (width 0.75) (layer F.Cu) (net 3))
 (segment (start 120.137799 101.900599) (end 120.137799 97.184601) (width 0.75) (layer F.Cu) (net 3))
 (segment (start 121.5136 103.2764) (end 120.137799 101.900599) (width 0.75) (layer F.Cu) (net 3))
 (segment (start 121.4628 95.2132) (end 126.9376 89.7384) (width 0.75) (layer F.Cu) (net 3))
 (segment (start 121.4628 95.8596) (end 121.4628 95.2132) (width 0.75) (layer F.Cu) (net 3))
 (segment (start 128.819601 114.307801) (end 130.557211 116.045411) (width 0.75) (layer F.Cu) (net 3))
 (segment (start 130.557211 116.045411) (end 141.204105 116.045411) (width 0.75) (layer F.Cu) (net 3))
 (segment (start 160.237401 99.909399) (end 158.9024 101.2444) (width 0.75) (layer B.Cu) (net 3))
 (segment (start 157.519398 109.945401) (end 147.304115 109.945401) (width 0.75) (layer F.Cu) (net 3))
 (segment (start 158.854399 108.6104) (end 157.519398 109.945401) (width 0.75) (layer F.Cu) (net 3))
 (segment (start 126.9376 86.5008) (end 129.5168 83.9216) (width 0.75) (layer F.Cu) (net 3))
 (segment (start 126.9376 89.7384) (end 126.9376 86.5008) (width 0.75) (layer F.Cu) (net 3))
 (segment (start 131.422 85.8268) (end 129.5168 83.9216) (width 0.75) (layer F.Cu) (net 3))
 (segment (start 136.6404 85.8268) (end 131.422 85.8268) (width 0.75) (layer F.Cu) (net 3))
 (segment (start 160.237401 89.371401) (end 159.9184 89.0524) (width 0.75) (layer B.Cu) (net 3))
 (segment (start 160.237401 99.909399) (end 160.237401 89.371401) (width 0.75) (layer B.Cu) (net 3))
 (segment (start 158.854399 101.292401) (end 158.9024 101.2444) (width 0.75) (layer B.Cu) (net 3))
 (segment (start 158.854399 108.6104) (end 158.854399 101.292401) (width 0.75) (layer B.Cu) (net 3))
 (segment (start 137.2464 85.2208) (end 136.6404 85.8268) (width 0.25) (layer F.Cu) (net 3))
 (segment (start 137.2464 84.1248) (end 137.2464 85.2208) (width 0.25) (layer F.Cu) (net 3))
 (segment (start 143.431474 112.595874) (end 144.042558 113.206958) (width 0.25) (layer F.Cu) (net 3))
 (segment (start 147.304115 109.945401) (end 144.042558 113.206958) (width 0.75) (layer F.Cu) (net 3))
 (segment (start 144.042558 113.206958) (end 141.204105 116.045411) (width 0.75) (layer F.Cu) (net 3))
 (segment (start 145.1356 114.3) (end 144.042558 113.206958) (width 0.25) (layer F.Cu) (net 3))
 (segment (start 147.2692 114.3) (end 145.1356 114.3) (width 0.25) (layer F.Cu) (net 3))
 (segment (start 150.2664 114.3) (end 151.6888 115.7224) (width 0.25) (layer F.Cu) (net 6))
 (segment (start 149.8092 114.3) (end 150.2664 114.3) (width 0.25) (layer F.Cu) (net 6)))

